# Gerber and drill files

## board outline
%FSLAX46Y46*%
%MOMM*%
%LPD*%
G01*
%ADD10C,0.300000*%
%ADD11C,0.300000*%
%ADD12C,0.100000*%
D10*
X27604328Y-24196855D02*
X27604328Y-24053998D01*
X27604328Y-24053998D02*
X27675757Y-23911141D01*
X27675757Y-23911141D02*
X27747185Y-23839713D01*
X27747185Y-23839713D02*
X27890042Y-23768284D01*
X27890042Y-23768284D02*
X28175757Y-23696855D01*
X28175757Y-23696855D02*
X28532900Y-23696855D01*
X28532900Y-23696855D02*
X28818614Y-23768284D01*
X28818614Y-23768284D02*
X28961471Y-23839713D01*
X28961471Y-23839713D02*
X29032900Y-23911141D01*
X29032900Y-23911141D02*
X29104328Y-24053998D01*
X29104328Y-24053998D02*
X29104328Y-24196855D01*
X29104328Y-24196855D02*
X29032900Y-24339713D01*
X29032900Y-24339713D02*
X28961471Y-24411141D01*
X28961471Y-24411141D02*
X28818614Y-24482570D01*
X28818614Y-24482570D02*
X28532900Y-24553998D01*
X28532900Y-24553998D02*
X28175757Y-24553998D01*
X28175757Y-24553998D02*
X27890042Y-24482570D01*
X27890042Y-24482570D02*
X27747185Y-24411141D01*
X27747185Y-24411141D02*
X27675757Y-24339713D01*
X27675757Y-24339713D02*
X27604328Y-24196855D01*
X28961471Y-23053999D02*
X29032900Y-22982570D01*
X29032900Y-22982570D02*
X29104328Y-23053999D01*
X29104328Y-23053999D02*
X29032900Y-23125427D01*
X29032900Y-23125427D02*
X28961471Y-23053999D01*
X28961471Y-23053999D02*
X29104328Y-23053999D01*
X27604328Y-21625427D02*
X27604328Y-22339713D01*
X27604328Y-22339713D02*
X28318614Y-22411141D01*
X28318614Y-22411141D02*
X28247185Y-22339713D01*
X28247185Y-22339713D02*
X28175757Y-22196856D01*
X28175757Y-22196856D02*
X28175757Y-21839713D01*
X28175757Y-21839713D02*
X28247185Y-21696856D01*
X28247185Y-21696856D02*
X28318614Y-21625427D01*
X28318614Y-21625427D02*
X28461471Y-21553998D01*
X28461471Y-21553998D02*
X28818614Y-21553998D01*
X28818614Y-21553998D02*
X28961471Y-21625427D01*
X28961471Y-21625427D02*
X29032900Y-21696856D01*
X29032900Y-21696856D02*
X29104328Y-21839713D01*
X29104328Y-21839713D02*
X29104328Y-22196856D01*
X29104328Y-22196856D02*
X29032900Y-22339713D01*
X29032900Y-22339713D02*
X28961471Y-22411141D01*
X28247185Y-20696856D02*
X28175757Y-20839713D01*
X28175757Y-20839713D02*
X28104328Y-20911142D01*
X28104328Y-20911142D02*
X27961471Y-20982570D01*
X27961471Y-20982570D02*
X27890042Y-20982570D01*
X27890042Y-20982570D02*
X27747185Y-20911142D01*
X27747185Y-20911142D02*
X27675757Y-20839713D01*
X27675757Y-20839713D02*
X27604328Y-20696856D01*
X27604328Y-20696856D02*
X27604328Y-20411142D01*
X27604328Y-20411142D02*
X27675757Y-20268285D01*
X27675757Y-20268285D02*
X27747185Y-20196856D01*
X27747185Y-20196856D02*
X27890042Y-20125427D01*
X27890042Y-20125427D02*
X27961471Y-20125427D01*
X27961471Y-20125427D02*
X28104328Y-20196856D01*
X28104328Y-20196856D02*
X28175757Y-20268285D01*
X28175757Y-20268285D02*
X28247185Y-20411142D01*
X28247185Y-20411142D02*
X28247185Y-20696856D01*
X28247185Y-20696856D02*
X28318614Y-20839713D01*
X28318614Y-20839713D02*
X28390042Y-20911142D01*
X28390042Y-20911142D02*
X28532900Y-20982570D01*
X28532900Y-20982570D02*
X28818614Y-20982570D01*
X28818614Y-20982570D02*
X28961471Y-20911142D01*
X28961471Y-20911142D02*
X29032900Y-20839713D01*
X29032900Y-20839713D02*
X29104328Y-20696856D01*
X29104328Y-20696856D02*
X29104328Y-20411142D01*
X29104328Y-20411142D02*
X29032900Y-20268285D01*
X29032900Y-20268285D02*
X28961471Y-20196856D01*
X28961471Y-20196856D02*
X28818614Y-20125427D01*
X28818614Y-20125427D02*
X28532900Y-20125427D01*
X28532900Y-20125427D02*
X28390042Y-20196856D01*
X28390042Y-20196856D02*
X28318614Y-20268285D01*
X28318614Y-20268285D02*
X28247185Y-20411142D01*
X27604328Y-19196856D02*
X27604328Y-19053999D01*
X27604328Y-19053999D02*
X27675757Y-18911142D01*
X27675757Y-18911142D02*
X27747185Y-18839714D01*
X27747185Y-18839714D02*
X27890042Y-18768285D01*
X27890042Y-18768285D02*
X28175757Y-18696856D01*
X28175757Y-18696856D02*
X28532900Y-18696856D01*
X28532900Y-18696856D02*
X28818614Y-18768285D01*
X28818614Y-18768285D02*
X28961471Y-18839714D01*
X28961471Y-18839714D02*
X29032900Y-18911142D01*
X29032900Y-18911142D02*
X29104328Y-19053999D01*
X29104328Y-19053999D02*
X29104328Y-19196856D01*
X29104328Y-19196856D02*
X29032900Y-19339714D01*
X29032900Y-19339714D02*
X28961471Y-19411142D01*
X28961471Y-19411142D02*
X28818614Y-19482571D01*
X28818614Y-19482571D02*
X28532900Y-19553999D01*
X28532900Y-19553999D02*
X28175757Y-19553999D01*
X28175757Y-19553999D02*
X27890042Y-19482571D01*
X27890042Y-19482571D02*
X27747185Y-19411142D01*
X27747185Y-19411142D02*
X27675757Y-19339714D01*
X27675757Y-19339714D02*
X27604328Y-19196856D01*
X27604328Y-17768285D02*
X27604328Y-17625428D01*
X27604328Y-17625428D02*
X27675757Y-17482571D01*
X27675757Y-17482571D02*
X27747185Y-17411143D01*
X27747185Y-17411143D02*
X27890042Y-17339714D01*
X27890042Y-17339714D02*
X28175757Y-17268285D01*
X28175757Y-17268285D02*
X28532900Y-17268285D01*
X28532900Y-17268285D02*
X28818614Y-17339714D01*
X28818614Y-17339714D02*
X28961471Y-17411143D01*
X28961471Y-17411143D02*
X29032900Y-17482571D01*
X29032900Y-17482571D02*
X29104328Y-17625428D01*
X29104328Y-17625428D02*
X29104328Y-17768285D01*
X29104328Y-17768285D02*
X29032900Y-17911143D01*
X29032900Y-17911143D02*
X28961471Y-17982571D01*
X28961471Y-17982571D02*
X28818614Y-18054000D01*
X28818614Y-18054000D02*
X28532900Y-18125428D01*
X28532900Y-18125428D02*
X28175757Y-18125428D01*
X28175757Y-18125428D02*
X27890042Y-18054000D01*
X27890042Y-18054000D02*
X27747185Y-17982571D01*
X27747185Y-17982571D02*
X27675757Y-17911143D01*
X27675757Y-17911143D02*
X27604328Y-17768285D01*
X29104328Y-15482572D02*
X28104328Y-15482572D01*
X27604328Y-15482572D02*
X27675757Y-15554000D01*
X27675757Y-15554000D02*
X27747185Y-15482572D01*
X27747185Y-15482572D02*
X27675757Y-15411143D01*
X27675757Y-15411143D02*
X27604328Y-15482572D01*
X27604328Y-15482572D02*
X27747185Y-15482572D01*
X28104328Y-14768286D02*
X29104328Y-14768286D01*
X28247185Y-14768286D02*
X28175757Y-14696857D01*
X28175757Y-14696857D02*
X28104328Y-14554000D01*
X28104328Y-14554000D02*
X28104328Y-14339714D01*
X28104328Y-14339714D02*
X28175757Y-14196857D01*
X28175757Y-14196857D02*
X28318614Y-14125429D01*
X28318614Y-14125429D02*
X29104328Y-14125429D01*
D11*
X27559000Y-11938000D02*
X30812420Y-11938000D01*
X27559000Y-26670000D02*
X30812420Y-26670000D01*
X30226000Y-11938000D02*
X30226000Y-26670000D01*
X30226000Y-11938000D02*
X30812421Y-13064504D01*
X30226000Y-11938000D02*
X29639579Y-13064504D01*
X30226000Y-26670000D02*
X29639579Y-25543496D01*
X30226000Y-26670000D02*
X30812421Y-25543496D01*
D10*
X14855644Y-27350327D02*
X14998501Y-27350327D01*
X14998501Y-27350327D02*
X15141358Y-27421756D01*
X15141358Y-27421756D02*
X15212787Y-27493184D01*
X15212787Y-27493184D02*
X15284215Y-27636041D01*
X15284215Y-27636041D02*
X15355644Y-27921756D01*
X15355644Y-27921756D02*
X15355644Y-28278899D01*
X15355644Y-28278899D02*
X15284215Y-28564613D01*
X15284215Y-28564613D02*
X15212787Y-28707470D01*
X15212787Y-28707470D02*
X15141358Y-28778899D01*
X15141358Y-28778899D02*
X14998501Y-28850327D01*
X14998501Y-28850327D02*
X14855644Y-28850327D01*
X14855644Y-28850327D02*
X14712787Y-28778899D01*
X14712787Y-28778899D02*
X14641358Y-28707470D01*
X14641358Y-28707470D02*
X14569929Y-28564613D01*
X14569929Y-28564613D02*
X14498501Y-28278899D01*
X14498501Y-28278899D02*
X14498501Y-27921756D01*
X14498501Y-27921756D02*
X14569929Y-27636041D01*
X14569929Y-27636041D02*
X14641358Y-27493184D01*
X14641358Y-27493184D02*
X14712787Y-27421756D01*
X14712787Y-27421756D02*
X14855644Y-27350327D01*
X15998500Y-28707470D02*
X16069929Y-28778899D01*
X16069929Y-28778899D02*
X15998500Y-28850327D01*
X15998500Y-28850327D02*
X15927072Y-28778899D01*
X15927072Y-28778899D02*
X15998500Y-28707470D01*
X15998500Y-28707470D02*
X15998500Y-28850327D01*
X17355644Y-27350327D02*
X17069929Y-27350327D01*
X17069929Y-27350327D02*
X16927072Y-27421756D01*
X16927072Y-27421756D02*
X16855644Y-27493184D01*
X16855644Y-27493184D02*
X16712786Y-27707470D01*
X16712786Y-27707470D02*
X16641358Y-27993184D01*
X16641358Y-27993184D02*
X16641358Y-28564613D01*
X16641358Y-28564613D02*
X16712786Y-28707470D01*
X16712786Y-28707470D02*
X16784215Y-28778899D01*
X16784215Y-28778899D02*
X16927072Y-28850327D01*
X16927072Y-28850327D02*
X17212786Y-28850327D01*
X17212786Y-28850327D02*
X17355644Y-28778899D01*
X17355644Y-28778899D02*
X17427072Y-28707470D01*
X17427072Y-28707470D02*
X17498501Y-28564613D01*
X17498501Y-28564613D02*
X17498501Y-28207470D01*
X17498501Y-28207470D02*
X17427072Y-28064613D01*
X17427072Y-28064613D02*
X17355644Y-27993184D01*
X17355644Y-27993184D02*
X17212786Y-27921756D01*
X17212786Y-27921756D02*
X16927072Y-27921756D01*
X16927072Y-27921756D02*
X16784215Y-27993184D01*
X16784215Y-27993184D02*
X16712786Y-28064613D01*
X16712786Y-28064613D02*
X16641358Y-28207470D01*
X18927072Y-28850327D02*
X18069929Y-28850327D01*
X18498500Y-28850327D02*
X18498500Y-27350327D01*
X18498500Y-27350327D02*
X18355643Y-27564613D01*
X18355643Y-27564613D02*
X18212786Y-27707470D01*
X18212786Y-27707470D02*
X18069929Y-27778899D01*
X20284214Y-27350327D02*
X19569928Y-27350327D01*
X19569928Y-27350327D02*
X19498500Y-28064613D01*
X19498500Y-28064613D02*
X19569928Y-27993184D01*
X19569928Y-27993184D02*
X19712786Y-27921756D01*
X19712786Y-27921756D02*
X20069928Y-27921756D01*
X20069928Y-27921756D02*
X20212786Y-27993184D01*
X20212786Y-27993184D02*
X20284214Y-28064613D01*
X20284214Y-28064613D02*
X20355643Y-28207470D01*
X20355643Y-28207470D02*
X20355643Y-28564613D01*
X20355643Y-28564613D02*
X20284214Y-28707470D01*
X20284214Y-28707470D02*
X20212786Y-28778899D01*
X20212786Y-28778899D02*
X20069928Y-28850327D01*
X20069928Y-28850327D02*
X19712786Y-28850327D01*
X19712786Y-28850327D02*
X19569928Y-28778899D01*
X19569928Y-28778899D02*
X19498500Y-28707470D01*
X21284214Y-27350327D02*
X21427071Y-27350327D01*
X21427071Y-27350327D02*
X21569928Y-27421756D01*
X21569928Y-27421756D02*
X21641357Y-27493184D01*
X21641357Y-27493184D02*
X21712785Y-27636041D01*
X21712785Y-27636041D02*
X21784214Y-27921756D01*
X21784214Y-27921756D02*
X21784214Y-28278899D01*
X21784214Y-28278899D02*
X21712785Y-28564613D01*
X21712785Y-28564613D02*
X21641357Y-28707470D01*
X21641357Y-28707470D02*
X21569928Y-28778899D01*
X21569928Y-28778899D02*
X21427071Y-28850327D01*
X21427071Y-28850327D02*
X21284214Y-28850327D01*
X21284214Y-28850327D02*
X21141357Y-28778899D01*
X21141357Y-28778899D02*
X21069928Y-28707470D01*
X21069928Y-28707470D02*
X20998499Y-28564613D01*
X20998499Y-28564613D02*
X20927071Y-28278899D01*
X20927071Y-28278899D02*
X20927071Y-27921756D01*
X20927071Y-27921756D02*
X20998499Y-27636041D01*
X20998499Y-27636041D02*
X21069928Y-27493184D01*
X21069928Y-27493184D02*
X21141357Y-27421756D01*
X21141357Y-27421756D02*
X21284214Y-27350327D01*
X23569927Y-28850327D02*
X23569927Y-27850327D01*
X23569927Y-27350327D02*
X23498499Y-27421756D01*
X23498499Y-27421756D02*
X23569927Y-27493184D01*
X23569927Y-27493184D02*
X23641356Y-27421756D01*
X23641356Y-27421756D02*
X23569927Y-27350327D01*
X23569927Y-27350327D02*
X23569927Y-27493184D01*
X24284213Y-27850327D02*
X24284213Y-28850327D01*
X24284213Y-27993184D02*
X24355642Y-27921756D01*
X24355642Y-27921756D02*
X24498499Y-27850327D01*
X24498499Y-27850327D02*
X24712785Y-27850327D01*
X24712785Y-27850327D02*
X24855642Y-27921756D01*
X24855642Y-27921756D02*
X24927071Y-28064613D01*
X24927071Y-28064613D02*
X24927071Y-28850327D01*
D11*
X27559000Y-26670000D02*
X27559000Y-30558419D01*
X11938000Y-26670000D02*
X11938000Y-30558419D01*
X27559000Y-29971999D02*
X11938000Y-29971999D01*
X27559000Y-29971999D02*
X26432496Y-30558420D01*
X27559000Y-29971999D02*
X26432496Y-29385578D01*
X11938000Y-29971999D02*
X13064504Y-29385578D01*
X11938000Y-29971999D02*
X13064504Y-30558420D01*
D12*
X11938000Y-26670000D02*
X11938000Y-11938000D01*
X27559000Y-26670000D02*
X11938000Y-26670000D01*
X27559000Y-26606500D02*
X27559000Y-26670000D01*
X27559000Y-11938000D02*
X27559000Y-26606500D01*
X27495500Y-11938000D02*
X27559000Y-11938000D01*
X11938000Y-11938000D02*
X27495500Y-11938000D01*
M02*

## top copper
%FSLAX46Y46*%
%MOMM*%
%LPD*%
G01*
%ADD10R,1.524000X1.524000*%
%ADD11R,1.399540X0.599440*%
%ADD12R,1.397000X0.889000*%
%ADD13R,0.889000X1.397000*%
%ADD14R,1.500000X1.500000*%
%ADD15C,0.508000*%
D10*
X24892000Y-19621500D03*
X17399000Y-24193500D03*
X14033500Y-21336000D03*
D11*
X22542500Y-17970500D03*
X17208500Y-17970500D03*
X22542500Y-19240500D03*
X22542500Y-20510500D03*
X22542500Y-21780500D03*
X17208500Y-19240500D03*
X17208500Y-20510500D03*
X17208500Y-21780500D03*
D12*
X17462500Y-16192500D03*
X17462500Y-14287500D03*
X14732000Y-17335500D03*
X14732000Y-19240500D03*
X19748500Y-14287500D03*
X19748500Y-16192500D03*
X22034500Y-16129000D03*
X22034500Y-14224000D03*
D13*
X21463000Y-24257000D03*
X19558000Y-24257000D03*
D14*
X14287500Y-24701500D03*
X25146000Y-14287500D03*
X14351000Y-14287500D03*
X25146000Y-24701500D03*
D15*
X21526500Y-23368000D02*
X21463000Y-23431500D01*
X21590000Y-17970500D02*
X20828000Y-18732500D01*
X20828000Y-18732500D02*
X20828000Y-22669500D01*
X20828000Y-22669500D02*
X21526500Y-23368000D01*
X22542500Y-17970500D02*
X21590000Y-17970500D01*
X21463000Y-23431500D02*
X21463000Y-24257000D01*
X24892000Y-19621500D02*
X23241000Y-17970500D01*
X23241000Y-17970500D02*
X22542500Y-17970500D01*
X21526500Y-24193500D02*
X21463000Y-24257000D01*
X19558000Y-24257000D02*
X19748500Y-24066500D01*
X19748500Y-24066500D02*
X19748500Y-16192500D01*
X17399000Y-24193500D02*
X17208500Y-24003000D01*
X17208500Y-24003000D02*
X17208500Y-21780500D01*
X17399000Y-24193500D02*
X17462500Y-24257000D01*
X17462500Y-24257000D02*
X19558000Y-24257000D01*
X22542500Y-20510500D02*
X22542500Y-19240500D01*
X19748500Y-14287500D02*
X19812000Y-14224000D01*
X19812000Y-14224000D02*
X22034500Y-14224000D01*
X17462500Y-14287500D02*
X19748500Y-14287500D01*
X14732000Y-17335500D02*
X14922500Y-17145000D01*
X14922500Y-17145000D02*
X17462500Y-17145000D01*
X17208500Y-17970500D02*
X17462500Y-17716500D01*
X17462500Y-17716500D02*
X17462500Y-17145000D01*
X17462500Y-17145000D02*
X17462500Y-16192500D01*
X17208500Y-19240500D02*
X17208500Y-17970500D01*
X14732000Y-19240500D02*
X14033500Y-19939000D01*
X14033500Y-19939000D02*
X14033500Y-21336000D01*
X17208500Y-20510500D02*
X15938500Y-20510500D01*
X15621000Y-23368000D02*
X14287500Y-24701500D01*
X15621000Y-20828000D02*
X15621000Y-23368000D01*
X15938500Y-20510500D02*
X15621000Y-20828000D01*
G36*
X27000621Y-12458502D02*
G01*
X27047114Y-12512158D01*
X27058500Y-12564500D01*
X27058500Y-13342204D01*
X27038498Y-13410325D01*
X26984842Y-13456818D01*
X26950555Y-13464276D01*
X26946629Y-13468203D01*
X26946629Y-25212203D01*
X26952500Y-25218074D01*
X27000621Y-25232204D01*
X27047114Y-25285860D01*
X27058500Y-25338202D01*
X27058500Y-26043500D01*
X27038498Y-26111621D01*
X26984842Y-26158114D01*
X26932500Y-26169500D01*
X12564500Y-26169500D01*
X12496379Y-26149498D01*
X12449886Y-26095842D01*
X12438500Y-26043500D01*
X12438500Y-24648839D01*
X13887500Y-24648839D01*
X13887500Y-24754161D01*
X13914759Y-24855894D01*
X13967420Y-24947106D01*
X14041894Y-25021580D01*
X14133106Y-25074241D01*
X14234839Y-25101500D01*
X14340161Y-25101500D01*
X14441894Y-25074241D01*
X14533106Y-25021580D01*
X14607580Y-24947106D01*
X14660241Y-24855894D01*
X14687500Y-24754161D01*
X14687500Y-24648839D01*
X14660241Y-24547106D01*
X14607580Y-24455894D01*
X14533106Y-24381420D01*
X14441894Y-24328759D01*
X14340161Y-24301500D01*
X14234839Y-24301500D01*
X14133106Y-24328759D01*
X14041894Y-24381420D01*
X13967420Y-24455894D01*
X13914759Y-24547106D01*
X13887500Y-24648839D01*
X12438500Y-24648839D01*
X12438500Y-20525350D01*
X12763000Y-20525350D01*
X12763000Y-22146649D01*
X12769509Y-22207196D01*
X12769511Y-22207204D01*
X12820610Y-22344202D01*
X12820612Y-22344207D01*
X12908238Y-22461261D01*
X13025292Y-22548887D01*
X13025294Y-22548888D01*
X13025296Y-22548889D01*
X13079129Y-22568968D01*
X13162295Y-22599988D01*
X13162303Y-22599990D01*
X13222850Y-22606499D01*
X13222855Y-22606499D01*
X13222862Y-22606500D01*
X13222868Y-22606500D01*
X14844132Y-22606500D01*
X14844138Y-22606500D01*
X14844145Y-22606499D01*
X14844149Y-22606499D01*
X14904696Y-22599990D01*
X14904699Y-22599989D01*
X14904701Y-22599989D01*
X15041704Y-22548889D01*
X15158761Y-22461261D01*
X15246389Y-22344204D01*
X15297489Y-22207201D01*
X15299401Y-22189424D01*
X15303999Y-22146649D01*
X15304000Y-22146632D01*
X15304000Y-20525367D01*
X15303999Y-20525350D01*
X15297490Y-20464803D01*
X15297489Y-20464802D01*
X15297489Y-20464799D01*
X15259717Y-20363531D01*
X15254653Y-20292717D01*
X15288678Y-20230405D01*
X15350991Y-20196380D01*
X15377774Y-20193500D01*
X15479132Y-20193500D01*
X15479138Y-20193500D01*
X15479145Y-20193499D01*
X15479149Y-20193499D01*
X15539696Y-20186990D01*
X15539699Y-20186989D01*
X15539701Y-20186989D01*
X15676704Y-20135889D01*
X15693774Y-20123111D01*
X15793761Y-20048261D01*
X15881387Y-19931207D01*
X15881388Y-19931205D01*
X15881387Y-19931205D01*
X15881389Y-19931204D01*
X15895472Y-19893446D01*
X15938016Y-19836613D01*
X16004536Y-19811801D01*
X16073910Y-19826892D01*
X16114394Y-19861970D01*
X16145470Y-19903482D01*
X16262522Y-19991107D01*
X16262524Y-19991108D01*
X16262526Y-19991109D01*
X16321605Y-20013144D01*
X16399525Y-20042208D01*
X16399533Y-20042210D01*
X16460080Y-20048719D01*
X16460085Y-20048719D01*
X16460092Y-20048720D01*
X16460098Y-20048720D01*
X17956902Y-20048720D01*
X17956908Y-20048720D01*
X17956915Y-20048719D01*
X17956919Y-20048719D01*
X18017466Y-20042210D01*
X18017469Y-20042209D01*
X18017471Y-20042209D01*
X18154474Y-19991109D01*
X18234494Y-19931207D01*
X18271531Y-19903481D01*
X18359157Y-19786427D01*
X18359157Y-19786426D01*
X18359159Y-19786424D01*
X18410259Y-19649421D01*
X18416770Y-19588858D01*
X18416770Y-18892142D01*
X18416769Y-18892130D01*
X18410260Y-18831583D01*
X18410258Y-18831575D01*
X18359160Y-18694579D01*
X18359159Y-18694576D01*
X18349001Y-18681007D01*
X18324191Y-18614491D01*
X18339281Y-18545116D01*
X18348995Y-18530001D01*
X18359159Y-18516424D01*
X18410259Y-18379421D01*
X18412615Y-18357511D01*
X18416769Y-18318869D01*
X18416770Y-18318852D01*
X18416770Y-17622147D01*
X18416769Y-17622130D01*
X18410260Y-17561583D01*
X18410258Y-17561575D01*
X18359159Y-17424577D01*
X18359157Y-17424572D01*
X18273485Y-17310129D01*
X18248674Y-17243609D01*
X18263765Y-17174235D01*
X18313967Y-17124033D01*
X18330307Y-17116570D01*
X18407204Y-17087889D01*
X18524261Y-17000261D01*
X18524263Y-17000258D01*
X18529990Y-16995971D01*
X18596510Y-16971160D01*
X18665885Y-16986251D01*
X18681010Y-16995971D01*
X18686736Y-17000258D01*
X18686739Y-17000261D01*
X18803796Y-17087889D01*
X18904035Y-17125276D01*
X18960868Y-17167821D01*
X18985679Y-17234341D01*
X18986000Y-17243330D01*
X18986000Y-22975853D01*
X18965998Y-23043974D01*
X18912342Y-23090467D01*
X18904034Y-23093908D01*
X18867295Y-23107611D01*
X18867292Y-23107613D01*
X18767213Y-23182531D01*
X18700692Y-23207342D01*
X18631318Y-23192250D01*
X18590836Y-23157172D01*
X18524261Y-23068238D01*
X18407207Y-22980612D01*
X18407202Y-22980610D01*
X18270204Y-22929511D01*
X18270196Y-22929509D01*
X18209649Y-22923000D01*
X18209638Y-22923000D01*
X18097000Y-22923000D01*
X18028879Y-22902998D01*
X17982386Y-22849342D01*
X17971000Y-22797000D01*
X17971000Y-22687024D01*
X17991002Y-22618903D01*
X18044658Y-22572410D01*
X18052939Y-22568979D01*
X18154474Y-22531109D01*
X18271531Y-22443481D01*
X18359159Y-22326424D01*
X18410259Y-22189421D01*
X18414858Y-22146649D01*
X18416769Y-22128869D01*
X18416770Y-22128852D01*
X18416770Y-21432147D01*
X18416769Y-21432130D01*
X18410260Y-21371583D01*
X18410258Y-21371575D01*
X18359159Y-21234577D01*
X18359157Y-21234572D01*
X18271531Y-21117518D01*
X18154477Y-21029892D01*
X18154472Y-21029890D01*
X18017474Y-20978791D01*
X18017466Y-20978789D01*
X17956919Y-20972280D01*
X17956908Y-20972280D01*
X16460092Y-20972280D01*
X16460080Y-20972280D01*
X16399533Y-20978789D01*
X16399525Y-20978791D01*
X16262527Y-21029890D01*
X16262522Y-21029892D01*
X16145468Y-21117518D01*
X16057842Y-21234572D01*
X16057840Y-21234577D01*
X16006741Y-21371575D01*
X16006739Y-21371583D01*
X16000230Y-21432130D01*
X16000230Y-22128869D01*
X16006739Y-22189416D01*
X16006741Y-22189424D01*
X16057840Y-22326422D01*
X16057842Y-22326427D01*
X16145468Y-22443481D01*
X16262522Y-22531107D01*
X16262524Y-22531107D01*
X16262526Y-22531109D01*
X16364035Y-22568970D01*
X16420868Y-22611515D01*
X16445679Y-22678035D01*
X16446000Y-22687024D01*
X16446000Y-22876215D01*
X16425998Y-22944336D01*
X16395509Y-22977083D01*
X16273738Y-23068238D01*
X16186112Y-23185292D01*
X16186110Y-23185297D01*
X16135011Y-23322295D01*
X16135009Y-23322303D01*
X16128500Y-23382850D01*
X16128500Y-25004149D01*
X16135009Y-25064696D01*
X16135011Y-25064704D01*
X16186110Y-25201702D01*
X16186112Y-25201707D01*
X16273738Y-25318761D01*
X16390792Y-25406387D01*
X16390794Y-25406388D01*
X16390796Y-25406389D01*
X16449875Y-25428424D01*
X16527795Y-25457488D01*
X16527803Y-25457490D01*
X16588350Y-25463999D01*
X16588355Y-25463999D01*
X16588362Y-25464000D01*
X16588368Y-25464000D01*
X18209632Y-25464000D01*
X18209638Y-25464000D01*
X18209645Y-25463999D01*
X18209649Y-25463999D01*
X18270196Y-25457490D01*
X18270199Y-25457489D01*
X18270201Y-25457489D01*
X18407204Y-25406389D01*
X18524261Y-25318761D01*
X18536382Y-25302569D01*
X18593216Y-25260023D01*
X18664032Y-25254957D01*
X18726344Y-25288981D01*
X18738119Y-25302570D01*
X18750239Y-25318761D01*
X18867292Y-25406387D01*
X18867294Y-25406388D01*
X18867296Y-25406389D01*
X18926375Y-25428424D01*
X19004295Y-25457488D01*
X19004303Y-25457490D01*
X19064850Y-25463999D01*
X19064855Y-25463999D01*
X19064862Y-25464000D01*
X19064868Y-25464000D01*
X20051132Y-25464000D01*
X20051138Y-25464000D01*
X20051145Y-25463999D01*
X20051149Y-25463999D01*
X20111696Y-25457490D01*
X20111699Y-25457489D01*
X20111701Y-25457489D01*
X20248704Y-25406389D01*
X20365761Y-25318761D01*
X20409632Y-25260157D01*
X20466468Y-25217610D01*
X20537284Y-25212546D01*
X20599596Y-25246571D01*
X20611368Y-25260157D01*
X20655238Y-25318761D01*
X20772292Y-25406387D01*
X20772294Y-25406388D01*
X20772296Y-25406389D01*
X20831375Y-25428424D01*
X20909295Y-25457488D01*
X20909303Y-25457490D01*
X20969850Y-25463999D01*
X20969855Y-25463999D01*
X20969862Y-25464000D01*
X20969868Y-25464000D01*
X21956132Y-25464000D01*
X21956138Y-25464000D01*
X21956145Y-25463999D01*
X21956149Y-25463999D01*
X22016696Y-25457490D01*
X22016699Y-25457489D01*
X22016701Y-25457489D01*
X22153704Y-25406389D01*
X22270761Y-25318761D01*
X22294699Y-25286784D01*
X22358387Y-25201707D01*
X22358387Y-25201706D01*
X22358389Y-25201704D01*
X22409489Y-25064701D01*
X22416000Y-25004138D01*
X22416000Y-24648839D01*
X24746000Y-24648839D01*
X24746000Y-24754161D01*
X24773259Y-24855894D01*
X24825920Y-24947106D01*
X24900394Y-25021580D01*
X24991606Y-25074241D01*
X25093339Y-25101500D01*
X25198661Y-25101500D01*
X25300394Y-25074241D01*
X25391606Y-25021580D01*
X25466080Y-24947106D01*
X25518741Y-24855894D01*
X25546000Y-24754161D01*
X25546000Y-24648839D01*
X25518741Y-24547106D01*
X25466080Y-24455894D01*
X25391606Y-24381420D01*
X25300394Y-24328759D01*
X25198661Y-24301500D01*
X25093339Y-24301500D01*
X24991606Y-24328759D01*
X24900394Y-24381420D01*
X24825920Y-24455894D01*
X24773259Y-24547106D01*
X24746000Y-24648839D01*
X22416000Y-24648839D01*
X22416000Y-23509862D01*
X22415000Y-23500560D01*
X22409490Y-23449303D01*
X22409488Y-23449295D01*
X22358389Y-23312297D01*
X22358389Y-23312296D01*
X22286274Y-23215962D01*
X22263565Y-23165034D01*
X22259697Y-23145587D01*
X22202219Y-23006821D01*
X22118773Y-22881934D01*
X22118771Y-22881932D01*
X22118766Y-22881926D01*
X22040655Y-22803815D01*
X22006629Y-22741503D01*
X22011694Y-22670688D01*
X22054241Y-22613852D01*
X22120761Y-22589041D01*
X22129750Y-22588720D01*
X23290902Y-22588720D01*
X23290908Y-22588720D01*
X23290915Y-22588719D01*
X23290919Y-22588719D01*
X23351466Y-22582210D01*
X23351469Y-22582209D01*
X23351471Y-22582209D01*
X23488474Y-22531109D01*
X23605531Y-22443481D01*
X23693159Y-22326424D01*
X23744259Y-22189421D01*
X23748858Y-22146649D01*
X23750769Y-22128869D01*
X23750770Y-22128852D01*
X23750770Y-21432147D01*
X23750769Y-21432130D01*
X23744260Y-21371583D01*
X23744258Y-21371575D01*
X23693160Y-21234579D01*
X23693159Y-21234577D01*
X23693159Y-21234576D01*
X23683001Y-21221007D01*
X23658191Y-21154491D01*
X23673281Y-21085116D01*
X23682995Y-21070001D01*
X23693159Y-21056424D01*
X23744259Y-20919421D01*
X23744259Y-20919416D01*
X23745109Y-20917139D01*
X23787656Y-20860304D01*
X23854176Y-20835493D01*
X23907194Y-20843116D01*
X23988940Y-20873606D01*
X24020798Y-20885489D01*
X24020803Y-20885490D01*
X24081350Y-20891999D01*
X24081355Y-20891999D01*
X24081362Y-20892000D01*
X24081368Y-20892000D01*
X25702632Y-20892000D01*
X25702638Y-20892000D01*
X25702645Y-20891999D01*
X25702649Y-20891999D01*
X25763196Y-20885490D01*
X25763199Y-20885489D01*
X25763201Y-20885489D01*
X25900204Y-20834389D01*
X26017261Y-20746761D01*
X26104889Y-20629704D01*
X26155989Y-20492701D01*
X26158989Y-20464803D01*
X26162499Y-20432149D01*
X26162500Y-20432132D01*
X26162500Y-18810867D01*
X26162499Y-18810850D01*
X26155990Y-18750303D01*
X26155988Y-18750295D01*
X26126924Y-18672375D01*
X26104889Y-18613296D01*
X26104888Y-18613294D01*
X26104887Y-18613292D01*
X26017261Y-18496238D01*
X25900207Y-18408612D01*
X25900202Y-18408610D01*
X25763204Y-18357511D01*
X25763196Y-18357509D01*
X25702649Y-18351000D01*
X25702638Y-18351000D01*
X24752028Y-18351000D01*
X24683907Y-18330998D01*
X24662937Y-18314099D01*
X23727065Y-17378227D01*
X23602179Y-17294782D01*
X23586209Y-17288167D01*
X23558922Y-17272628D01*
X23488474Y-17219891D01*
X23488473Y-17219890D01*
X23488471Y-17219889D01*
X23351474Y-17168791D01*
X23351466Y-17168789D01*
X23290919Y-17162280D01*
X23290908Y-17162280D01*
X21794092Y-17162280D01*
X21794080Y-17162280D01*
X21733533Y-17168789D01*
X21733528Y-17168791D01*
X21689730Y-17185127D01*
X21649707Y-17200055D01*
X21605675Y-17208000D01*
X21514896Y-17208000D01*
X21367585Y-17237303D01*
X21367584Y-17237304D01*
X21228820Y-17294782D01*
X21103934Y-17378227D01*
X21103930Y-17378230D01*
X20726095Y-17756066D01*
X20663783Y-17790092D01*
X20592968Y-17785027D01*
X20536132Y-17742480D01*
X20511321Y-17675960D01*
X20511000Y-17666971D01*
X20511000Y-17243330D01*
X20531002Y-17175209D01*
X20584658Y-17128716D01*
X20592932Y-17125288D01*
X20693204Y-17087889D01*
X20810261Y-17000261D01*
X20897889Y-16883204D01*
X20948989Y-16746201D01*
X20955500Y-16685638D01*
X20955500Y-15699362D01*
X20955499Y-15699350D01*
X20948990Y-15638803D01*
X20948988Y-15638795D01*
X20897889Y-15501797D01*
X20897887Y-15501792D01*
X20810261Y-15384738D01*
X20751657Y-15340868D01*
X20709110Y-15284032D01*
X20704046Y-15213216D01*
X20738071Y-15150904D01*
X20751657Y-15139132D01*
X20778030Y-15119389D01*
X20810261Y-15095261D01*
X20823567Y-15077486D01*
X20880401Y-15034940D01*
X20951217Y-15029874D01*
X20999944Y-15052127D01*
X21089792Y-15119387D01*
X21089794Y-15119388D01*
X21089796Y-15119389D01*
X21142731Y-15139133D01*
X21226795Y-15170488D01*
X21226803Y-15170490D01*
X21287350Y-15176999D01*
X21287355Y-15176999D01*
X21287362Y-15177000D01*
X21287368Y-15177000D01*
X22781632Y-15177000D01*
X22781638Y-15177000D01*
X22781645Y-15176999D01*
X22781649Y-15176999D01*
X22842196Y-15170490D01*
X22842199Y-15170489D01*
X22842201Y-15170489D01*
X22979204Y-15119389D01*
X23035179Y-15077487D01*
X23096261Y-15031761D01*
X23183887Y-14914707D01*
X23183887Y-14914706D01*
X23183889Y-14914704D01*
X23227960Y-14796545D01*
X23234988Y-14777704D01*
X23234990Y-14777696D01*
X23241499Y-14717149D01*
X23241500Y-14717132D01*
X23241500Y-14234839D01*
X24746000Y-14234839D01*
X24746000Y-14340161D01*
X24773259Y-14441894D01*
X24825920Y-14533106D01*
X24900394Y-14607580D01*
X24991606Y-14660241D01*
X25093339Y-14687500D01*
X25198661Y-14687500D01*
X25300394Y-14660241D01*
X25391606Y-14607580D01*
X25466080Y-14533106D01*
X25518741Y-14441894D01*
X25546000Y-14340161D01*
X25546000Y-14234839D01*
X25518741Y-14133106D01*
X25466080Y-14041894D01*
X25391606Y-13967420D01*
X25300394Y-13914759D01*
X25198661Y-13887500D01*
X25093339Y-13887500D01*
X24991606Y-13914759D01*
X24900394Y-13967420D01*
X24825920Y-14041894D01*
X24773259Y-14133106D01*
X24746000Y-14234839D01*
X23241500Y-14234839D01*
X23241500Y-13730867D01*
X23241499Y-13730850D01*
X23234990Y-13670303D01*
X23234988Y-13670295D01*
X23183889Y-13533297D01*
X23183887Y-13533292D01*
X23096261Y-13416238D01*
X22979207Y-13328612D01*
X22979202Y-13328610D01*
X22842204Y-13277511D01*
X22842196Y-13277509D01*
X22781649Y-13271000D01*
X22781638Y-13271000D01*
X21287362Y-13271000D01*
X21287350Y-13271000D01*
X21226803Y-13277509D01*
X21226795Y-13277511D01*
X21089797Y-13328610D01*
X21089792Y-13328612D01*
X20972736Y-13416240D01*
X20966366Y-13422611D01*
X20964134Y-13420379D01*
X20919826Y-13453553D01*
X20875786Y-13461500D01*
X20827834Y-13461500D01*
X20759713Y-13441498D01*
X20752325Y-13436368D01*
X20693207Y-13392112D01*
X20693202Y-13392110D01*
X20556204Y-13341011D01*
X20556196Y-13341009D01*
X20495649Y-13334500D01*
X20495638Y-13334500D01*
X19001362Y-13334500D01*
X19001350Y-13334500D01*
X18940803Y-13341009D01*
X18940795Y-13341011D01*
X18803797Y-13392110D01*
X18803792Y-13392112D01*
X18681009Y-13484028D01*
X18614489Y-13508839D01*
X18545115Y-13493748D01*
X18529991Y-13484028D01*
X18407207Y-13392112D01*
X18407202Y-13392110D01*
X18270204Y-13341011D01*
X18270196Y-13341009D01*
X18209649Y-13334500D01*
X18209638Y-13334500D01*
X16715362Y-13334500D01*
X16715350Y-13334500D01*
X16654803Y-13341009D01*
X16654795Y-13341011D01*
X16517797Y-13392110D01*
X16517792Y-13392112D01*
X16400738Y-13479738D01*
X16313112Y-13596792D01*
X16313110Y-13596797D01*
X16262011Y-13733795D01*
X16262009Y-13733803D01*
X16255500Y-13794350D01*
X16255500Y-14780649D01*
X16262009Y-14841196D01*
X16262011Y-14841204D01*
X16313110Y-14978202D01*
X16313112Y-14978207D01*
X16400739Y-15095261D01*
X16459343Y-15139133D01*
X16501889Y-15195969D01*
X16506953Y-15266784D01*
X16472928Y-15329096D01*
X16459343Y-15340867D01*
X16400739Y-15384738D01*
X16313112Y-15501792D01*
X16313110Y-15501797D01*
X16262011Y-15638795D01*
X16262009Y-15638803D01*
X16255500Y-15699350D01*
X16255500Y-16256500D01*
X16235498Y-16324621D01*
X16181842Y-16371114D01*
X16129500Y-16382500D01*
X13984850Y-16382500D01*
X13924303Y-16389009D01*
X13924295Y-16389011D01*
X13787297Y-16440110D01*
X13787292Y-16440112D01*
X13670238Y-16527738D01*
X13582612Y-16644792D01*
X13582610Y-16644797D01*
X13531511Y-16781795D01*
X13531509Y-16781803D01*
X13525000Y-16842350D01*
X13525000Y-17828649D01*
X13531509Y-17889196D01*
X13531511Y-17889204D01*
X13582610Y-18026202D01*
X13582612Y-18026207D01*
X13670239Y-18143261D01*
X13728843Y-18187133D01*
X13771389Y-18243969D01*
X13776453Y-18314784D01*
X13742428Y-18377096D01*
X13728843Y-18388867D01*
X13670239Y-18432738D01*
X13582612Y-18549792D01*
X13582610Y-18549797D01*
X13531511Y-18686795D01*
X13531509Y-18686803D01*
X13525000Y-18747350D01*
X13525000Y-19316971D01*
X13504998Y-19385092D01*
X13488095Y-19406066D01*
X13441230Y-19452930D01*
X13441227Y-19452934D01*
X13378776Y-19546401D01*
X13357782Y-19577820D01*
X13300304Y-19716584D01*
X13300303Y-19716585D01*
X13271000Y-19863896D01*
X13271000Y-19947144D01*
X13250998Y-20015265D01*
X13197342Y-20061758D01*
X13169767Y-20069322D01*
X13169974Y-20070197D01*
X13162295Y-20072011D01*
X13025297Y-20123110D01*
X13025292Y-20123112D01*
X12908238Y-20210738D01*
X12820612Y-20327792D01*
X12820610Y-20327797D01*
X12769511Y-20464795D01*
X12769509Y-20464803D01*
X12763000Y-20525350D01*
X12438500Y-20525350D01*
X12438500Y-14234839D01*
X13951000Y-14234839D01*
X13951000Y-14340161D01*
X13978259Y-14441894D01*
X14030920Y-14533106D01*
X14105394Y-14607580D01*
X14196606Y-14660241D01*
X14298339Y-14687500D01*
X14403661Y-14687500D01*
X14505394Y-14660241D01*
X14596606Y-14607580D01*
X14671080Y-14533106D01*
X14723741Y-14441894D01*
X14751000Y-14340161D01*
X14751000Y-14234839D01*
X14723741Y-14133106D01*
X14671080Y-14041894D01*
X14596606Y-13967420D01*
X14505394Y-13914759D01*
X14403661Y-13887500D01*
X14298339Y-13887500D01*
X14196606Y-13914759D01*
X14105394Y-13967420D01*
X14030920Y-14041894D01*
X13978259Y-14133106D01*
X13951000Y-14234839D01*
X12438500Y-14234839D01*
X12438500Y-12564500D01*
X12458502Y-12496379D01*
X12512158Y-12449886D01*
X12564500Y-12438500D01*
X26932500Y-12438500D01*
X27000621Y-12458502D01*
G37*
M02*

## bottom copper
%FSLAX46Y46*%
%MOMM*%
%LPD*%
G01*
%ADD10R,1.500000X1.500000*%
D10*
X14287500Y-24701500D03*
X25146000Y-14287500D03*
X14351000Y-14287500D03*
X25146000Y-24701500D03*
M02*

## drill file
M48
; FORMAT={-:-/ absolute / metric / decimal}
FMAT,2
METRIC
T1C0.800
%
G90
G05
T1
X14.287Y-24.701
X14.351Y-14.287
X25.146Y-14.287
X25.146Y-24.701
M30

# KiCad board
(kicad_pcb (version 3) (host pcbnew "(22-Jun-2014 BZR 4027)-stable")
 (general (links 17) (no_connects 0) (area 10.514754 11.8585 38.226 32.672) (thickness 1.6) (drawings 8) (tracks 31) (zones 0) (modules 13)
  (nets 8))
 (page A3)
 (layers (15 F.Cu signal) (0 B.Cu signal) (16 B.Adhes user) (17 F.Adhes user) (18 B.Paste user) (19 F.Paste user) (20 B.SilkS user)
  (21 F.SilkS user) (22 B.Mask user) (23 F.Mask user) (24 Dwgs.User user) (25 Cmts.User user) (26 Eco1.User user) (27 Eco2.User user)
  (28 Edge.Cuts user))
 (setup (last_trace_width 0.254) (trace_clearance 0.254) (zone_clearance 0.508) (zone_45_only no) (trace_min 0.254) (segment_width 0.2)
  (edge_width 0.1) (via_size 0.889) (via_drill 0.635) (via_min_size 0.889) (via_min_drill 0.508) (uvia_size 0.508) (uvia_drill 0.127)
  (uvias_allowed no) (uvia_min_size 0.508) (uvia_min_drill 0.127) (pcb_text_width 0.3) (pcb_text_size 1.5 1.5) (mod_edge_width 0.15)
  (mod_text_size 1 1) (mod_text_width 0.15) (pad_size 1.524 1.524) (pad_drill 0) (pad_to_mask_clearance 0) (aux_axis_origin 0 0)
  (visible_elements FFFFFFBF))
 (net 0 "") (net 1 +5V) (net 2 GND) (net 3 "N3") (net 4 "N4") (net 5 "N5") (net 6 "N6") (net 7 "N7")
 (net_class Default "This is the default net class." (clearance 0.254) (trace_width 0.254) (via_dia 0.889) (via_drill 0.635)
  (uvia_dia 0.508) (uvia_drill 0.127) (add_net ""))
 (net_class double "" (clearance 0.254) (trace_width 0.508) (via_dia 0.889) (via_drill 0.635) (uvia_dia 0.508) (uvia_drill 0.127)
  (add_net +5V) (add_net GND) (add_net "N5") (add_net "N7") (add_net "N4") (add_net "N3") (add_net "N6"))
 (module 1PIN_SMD (layer F.Cu) (at 24.892 19.6215)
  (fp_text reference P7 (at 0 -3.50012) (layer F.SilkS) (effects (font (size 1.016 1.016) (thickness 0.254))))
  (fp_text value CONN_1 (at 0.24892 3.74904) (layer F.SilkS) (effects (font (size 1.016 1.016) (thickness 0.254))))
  (pad 1 smd rect (at 0 0) (size 1.524 1.524) (layers F.Cu F.Paste F.SilkS F.Mask) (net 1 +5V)))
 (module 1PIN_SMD (layer F.Cu) (at 17.399 24.1935)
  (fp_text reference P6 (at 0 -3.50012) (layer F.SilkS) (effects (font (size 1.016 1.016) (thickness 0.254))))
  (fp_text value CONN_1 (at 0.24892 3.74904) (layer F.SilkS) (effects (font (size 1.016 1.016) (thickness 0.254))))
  (pad 1 smd rect (at 0 0) (size 1.524 1.524) (layers F.Cu F.Paste F.SilkS F.Mask) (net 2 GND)))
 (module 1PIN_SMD (layer F.Cu) (at 14.0335 21.336)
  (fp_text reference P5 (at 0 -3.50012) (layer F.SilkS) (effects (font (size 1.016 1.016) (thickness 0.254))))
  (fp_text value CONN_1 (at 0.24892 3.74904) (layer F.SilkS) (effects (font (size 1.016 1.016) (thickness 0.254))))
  (pad 1 smd rect (at 0 0) (size 1.524 1.524) (layers F.Cu F.Paste F.SilkS F.Mask) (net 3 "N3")))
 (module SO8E (layer F.Cu) (at 19.8755 19.8755 270)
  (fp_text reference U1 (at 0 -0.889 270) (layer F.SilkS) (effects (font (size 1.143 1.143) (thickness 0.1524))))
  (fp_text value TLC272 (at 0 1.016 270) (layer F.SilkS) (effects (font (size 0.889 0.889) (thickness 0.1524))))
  (pad 8 smd rect (at -1.905 -2.667 270) (size 0.59944 1.39954) (layers F.Cu F.Paste F.Mask) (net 1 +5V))
  (pad 1 smd rect (at -1.905 2.667 270) (size 0.59944 1.39954) (layers F.Cu F.Paste F.Mask) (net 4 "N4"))
  (pad 7 smd rect (at -0.635 -2.667 270) (size 0.59944 1.39954) (layers F.Cu F.Paste F.Mask) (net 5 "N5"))
  (pad 6 smd rect (at 0.635 -2.667 270) (size 0.59944 1.39954) (layers F.Cu F.Paste F.Mask) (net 5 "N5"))
  (pad 5 smd rect (at 1.905 -2.667 270) (size 0.59944 1.39954) (layers F.Cu F.Paste F.Mask))
  (pad 2 smd rect (at -0.635 2.667 270) (size 0.59944 1.39954) (layers F.Cu F.Paste F.Mask) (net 4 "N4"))
  (pad 3 smd rect (at 0.635 2.667 270) (size 0.59944 1.39954) (layers F.Cu F.Paste F.Mask) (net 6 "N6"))
  (pad 4 smd rect (at 1.905 2.667 270) (size 0.59944 1.39954) (layers F.Cu F.Paste F.Mask) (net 2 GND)))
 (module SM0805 (layer F.Cu) (at 17.4625 15.24 90)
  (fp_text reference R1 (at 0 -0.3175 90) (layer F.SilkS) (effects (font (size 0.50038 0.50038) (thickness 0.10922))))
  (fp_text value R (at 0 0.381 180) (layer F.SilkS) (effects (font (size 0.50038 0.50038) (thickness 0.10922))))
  (pad 1 smd rect (at -0.9525 0 90) (size 0.889 1.397) (layers F.Cu F.Paste F.Mask) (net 4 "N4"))
  (pad 2 smd rect (at 0.9525 0 90) (size 0.889 1.397) (layers F.Cu F.Paste F.Mask) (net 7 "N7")))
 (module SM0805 (layer F.Cu) (at 14.732 18.288 270)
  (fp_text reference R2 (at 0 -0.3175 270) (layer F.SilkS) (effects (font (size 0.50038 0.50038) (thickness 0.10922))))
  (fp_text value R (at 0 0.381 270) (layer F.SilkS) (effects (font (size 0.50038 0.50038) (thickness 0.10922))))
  (pad 1 smd rect (at -0.9525 0 270) (size 0.889 1.397) (layers F.Cu F.Paste F.Mask) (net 4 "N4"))
  (pad 2 smd rect (at 0.9525 0 270) (size 0.889 1.397) (layers F.Cu F.Paste F.Mask) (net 3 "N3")))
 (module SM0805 (layer F.Cu) (at 19.7485 15.24 270)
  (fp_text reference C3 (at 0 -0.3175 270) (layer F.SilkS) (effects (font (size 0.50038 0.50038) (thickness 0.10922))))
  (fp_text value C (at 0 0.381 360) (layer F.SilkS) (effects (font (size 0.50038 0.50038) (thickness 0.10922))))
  (pad 1 smd rect (at -0.9525 0 270) (size 0.889 1.397) (layers F.Cu F.Paste F.Mask) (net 7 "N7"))
  (pad 2 smd rect (at 0.9525 0 270) (size 0.889 1.397) (layers F.Cu F.Paste F.Mask) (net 2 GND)))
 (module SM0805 (layer F.Cu) (at 22.0345 15.1765 90)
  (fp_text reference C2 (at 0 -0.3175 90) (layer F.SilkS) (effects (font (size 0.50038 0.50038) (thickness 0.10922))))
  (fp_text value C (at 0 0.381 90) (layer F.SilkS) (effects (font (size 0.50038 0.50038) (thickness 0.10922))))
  (pad 1 smd rect (at -0.9525 0 90) (size 0.889 1.397) (layers F.Cu F.Paste F.Mask) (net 6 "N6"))
  (pad 2 smd rect (at 0.9525 0 90) (size 0.889 1.397) (layers F.Cu F.Paste F.Mask) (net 7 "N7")))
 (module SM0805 (layer F.Cu) (at 20.5105 24.257 180)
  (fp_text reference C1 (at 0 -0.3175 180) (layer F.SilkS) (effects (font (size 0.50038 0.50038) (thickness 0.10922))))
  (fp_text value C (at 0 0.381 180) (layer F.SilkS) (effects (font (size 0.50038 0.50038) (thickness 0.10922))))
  (pad 1 smd rect (at -0.9525 0 180) (size 0.889 1.397) (layers F.Cu F.Paste F.Mask) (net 1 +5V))
  (pad 2 smd rect (at 0.9525 0 180) (size 0.889 1.397) (layers F.Cu F.Paste F.Mask) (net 2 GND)))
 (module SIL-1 (layer F.Cu) (at 14.2875 24.7015)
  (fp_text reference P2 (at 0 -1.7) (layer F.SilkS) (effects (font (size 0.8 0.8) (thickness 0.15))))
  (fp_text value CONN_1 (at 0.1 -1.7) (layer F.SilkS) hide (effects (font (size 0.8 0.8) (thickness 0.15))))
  (pad 1 thru_hole rect (at 0 0) (size 1.5 1.5) (drill 0.8) (layers *.Cu *.Mask F.SilkS) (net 6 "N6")))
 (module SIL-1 (layer F.Cu) (at 25.146 14.2875)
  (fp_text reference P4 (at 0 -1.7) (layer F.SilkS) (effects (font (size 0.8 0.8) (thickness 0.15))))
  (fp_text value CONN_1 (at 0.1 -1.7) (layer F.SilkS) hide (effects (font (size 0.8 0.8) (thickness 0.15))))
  (pad 1 thru_hole rect (at 0 0) (size 1.5 1.5) (drill 0.8) (layers *.Cu *.Mask F.SilkS) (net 6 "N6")))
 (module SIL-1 (layer F.Cu) (at 14.351 14.2875)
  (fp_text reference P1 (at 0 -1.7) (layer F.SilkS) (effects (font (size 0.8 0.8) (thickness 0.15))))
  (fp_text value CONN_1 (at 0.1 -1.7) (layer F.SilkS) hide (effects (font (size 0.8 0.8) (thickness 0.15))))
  (pad 1 thru_hole rect (at 0 0) (size 1.5 1.5) (drill 0.8) (layers *.Cu *.Mask F.SilkS) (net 6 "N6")))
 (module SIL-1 (layer F.Cu) (at 25.146 24.7015)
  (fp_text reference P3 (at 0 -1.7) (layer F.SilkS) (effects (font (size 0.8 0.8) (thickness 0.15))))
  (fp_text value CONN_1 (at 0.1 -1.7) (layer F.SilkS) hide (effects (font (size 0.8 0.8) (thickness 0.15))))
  (pad 1 thru_hole rect (at 0 0) (size 1.5 1.5) (drill 0.8) (layers *.Cu *.Mask F.SilkS) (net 6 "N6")))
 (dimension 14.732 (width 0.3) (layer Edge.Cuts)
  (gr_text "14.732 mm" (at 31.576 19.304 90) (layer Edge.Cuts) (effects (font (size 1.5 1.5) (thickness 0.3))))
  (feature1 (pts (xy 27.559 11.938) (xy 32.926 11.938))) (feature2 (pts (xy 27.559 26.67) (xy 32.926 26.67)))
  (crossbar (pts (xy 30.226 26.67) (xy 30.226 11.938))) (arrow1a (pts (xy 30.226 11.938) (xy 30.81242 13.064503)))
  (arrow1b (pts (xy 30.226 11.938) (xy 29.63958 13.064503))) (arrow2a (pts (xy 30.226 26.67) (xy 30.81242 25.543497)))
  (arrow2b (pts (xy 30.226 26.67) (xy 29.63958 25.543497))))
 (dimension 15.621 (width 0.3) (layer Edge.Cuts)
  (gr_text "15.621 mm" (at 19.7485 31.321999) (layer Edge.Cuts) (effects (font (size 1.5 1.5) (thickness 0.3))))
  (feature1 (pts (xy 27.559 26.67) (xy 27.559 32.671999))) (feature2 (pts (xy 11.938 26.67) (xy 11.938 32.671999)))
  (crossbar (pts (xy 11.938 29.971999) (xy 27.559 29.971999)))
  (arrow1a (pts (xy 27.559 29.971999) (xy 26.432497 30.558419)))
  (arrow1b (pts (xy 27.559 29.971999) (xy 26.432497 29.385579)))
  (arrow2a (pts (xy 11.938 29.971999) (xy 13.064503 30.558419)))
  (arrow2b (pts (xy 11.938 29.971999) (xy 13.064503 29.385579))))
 (gr_line (start 11.938 26.67) (end 11.938 11.938) (angle 90) (layer Edge.Cuts) (width 0.1))
 (gr_line (start 27.559 26.67) (end 11.938 26.67) (angle 90) (layer Edge.Cuts) (width 0.1))
 (gr_line (start 27.559 26.6065) (end 27.559 26.67) (angle 90) (layer Edge.Cuts) (width 0.1))
 (gr_line (start 27.559 11.938) (end 27.559 26.6065) (angle 90) (layer Edge.Cuts) (width 0.1))
 (gr_line (start 27.4955 11.938) (end 27.559 11.938) (angle 90) (layer Edge.Cuts) (width 0.1))
 (gr_line (start 11.938 11.938) (end 27.4955 11.938) (angle 90) (layer Edge.Cuts) (width 0.1))
 (segment (start 21.5265 23.368) (end 21.463 23.4315) (width 0.508) (layer F.Cu) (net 1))
 (segment (start 21.59 17.9705) (end 20.828 18.7325) (width 0.508) (layer F.Cu) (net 1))
 (segment (start 20.828 18.7325) (end 20.828 22.6695) (width 0.508) (layer F.Cu) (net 1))
 (segment (start 20.828 22.6695) (end 21.5265 23.368) (width 0.508) (layer F.Cu) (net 1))
 (segment (start 22.5425 17.9705) (end 21.59 17.9705) (width 0.508) (layer F.Cu) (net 1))
 (segment (start 21.463 23.4315) (end 21.463 24.257) (width 0.508) (layer F.Cu) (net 1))
 (segment (start 24.892 19.6215) (end 23.241 17.9705) (width 0.508) (layer F.Cu) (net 1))
 (segment (start 23.241 17.9705) (end 22.5425 17.9705) (width 0.508) (layer F.Cu) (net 1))
 (segment (start 21.5265 24.1935) (end 21.463 24.257) (width 0.508) (layer F.Cu) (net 1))
 (segment (start 19.558 24.257) (end 19.7485 24.0665) (width 0.508) (layer F.Cu) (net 2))
 (segment (start 19.7485 24.0665) (end 19.7485 16.1925) (width 0.508) (layer F.Cu) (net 2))
 (segment (start 17.399 24.1935) (end 17.2085 24.003) (width 0.508) (layer F.Cu) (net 2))
 (segment (start 17.2085 24.003) (end 17.2085 21.7805) (width 0.508) (layer F.Cu) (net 2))
 (segment (start 17.399 24.1935) (end 17.4625 24.257) (width 0.508) (layer F.Cu) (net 2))
 (segment (start 17.4625 24.257) (end 19.558 24.257) (width 0.508) (layer F.Cu) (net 2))
 (segment (start 22.5425 20.5105) (end 22.5425 19.2405) (width 0.508) (layer F.Cu) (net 5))
 (segment (start 19.7485 14.2875) (end 19.812 14.224) (width 0.508) (layer F.Cu) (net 7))
 (segment (start 19.812 14.224) (end 22.0345 14.224) (width 0.508) (layer F.Cu) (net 7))
 (segment (start 17.4625 14.2875) (end 19.7485 14.2875) (width 0.508) (layer F.Cu) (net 7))
 (segment (start 14.732 17.3355) (end 14.9225 17.145) (width 0.508) (layer F.Cu) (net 4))
 (segment (start 14.9225 17.145) (end 17.4625 17.145) (width 0.508) (layer F.Cu) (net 4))
 (segment (start 17.2085 17.9705) (end 17.4625 17.7165) (width 0.508) (layer F.Cu) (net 4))
 (segment (start 17.4625 17.7165) (end 17.4625 17.145) (width 0.508) (layer F.Cu) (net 4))
 (segment (start 17.4625 17.145) (end 17.4625 16.1925) (width 0.508) (layer F.Cu) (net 4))
 (segment (start 17.2085 19.2405) (end 17.2085 17.9705) (width 0.508) (layer F.Cu) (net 4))
 (segment (start 14.732 19.2405) (end 14.0335 19.939) (width 0.508) (layer F.Cu) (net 3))
 (segment (start 14.0335 19.939) (end 14.0335 21.336) (width 0.508) (layer F.Cu) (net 3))
 (segment (start 17.2085 20.5105) (end 15.9385 20.5105) (width 0.508) (layer F.Cu) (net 6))
 (segment (start 15.621 23.368) (end 14.2875 24.7015) (width 0.508) (layer F.Cu) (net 6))
 (segment (start 15.621 20.828) (end 15.621 23.368) (width 0.508) (layer F.Cu) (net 6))
 (segment (start 15.9385 20.5105) (end 15.621 20.828) (width 0.508) (layer F.Cu) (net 6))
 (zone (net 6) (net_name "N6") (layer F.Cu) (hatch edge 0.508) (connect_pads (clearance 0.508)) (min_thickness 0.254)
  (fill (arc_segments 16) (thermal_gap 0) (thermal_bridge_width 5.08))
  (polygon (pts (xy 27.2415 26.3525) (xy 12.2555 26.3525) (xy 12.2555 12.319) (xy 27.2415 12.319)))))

